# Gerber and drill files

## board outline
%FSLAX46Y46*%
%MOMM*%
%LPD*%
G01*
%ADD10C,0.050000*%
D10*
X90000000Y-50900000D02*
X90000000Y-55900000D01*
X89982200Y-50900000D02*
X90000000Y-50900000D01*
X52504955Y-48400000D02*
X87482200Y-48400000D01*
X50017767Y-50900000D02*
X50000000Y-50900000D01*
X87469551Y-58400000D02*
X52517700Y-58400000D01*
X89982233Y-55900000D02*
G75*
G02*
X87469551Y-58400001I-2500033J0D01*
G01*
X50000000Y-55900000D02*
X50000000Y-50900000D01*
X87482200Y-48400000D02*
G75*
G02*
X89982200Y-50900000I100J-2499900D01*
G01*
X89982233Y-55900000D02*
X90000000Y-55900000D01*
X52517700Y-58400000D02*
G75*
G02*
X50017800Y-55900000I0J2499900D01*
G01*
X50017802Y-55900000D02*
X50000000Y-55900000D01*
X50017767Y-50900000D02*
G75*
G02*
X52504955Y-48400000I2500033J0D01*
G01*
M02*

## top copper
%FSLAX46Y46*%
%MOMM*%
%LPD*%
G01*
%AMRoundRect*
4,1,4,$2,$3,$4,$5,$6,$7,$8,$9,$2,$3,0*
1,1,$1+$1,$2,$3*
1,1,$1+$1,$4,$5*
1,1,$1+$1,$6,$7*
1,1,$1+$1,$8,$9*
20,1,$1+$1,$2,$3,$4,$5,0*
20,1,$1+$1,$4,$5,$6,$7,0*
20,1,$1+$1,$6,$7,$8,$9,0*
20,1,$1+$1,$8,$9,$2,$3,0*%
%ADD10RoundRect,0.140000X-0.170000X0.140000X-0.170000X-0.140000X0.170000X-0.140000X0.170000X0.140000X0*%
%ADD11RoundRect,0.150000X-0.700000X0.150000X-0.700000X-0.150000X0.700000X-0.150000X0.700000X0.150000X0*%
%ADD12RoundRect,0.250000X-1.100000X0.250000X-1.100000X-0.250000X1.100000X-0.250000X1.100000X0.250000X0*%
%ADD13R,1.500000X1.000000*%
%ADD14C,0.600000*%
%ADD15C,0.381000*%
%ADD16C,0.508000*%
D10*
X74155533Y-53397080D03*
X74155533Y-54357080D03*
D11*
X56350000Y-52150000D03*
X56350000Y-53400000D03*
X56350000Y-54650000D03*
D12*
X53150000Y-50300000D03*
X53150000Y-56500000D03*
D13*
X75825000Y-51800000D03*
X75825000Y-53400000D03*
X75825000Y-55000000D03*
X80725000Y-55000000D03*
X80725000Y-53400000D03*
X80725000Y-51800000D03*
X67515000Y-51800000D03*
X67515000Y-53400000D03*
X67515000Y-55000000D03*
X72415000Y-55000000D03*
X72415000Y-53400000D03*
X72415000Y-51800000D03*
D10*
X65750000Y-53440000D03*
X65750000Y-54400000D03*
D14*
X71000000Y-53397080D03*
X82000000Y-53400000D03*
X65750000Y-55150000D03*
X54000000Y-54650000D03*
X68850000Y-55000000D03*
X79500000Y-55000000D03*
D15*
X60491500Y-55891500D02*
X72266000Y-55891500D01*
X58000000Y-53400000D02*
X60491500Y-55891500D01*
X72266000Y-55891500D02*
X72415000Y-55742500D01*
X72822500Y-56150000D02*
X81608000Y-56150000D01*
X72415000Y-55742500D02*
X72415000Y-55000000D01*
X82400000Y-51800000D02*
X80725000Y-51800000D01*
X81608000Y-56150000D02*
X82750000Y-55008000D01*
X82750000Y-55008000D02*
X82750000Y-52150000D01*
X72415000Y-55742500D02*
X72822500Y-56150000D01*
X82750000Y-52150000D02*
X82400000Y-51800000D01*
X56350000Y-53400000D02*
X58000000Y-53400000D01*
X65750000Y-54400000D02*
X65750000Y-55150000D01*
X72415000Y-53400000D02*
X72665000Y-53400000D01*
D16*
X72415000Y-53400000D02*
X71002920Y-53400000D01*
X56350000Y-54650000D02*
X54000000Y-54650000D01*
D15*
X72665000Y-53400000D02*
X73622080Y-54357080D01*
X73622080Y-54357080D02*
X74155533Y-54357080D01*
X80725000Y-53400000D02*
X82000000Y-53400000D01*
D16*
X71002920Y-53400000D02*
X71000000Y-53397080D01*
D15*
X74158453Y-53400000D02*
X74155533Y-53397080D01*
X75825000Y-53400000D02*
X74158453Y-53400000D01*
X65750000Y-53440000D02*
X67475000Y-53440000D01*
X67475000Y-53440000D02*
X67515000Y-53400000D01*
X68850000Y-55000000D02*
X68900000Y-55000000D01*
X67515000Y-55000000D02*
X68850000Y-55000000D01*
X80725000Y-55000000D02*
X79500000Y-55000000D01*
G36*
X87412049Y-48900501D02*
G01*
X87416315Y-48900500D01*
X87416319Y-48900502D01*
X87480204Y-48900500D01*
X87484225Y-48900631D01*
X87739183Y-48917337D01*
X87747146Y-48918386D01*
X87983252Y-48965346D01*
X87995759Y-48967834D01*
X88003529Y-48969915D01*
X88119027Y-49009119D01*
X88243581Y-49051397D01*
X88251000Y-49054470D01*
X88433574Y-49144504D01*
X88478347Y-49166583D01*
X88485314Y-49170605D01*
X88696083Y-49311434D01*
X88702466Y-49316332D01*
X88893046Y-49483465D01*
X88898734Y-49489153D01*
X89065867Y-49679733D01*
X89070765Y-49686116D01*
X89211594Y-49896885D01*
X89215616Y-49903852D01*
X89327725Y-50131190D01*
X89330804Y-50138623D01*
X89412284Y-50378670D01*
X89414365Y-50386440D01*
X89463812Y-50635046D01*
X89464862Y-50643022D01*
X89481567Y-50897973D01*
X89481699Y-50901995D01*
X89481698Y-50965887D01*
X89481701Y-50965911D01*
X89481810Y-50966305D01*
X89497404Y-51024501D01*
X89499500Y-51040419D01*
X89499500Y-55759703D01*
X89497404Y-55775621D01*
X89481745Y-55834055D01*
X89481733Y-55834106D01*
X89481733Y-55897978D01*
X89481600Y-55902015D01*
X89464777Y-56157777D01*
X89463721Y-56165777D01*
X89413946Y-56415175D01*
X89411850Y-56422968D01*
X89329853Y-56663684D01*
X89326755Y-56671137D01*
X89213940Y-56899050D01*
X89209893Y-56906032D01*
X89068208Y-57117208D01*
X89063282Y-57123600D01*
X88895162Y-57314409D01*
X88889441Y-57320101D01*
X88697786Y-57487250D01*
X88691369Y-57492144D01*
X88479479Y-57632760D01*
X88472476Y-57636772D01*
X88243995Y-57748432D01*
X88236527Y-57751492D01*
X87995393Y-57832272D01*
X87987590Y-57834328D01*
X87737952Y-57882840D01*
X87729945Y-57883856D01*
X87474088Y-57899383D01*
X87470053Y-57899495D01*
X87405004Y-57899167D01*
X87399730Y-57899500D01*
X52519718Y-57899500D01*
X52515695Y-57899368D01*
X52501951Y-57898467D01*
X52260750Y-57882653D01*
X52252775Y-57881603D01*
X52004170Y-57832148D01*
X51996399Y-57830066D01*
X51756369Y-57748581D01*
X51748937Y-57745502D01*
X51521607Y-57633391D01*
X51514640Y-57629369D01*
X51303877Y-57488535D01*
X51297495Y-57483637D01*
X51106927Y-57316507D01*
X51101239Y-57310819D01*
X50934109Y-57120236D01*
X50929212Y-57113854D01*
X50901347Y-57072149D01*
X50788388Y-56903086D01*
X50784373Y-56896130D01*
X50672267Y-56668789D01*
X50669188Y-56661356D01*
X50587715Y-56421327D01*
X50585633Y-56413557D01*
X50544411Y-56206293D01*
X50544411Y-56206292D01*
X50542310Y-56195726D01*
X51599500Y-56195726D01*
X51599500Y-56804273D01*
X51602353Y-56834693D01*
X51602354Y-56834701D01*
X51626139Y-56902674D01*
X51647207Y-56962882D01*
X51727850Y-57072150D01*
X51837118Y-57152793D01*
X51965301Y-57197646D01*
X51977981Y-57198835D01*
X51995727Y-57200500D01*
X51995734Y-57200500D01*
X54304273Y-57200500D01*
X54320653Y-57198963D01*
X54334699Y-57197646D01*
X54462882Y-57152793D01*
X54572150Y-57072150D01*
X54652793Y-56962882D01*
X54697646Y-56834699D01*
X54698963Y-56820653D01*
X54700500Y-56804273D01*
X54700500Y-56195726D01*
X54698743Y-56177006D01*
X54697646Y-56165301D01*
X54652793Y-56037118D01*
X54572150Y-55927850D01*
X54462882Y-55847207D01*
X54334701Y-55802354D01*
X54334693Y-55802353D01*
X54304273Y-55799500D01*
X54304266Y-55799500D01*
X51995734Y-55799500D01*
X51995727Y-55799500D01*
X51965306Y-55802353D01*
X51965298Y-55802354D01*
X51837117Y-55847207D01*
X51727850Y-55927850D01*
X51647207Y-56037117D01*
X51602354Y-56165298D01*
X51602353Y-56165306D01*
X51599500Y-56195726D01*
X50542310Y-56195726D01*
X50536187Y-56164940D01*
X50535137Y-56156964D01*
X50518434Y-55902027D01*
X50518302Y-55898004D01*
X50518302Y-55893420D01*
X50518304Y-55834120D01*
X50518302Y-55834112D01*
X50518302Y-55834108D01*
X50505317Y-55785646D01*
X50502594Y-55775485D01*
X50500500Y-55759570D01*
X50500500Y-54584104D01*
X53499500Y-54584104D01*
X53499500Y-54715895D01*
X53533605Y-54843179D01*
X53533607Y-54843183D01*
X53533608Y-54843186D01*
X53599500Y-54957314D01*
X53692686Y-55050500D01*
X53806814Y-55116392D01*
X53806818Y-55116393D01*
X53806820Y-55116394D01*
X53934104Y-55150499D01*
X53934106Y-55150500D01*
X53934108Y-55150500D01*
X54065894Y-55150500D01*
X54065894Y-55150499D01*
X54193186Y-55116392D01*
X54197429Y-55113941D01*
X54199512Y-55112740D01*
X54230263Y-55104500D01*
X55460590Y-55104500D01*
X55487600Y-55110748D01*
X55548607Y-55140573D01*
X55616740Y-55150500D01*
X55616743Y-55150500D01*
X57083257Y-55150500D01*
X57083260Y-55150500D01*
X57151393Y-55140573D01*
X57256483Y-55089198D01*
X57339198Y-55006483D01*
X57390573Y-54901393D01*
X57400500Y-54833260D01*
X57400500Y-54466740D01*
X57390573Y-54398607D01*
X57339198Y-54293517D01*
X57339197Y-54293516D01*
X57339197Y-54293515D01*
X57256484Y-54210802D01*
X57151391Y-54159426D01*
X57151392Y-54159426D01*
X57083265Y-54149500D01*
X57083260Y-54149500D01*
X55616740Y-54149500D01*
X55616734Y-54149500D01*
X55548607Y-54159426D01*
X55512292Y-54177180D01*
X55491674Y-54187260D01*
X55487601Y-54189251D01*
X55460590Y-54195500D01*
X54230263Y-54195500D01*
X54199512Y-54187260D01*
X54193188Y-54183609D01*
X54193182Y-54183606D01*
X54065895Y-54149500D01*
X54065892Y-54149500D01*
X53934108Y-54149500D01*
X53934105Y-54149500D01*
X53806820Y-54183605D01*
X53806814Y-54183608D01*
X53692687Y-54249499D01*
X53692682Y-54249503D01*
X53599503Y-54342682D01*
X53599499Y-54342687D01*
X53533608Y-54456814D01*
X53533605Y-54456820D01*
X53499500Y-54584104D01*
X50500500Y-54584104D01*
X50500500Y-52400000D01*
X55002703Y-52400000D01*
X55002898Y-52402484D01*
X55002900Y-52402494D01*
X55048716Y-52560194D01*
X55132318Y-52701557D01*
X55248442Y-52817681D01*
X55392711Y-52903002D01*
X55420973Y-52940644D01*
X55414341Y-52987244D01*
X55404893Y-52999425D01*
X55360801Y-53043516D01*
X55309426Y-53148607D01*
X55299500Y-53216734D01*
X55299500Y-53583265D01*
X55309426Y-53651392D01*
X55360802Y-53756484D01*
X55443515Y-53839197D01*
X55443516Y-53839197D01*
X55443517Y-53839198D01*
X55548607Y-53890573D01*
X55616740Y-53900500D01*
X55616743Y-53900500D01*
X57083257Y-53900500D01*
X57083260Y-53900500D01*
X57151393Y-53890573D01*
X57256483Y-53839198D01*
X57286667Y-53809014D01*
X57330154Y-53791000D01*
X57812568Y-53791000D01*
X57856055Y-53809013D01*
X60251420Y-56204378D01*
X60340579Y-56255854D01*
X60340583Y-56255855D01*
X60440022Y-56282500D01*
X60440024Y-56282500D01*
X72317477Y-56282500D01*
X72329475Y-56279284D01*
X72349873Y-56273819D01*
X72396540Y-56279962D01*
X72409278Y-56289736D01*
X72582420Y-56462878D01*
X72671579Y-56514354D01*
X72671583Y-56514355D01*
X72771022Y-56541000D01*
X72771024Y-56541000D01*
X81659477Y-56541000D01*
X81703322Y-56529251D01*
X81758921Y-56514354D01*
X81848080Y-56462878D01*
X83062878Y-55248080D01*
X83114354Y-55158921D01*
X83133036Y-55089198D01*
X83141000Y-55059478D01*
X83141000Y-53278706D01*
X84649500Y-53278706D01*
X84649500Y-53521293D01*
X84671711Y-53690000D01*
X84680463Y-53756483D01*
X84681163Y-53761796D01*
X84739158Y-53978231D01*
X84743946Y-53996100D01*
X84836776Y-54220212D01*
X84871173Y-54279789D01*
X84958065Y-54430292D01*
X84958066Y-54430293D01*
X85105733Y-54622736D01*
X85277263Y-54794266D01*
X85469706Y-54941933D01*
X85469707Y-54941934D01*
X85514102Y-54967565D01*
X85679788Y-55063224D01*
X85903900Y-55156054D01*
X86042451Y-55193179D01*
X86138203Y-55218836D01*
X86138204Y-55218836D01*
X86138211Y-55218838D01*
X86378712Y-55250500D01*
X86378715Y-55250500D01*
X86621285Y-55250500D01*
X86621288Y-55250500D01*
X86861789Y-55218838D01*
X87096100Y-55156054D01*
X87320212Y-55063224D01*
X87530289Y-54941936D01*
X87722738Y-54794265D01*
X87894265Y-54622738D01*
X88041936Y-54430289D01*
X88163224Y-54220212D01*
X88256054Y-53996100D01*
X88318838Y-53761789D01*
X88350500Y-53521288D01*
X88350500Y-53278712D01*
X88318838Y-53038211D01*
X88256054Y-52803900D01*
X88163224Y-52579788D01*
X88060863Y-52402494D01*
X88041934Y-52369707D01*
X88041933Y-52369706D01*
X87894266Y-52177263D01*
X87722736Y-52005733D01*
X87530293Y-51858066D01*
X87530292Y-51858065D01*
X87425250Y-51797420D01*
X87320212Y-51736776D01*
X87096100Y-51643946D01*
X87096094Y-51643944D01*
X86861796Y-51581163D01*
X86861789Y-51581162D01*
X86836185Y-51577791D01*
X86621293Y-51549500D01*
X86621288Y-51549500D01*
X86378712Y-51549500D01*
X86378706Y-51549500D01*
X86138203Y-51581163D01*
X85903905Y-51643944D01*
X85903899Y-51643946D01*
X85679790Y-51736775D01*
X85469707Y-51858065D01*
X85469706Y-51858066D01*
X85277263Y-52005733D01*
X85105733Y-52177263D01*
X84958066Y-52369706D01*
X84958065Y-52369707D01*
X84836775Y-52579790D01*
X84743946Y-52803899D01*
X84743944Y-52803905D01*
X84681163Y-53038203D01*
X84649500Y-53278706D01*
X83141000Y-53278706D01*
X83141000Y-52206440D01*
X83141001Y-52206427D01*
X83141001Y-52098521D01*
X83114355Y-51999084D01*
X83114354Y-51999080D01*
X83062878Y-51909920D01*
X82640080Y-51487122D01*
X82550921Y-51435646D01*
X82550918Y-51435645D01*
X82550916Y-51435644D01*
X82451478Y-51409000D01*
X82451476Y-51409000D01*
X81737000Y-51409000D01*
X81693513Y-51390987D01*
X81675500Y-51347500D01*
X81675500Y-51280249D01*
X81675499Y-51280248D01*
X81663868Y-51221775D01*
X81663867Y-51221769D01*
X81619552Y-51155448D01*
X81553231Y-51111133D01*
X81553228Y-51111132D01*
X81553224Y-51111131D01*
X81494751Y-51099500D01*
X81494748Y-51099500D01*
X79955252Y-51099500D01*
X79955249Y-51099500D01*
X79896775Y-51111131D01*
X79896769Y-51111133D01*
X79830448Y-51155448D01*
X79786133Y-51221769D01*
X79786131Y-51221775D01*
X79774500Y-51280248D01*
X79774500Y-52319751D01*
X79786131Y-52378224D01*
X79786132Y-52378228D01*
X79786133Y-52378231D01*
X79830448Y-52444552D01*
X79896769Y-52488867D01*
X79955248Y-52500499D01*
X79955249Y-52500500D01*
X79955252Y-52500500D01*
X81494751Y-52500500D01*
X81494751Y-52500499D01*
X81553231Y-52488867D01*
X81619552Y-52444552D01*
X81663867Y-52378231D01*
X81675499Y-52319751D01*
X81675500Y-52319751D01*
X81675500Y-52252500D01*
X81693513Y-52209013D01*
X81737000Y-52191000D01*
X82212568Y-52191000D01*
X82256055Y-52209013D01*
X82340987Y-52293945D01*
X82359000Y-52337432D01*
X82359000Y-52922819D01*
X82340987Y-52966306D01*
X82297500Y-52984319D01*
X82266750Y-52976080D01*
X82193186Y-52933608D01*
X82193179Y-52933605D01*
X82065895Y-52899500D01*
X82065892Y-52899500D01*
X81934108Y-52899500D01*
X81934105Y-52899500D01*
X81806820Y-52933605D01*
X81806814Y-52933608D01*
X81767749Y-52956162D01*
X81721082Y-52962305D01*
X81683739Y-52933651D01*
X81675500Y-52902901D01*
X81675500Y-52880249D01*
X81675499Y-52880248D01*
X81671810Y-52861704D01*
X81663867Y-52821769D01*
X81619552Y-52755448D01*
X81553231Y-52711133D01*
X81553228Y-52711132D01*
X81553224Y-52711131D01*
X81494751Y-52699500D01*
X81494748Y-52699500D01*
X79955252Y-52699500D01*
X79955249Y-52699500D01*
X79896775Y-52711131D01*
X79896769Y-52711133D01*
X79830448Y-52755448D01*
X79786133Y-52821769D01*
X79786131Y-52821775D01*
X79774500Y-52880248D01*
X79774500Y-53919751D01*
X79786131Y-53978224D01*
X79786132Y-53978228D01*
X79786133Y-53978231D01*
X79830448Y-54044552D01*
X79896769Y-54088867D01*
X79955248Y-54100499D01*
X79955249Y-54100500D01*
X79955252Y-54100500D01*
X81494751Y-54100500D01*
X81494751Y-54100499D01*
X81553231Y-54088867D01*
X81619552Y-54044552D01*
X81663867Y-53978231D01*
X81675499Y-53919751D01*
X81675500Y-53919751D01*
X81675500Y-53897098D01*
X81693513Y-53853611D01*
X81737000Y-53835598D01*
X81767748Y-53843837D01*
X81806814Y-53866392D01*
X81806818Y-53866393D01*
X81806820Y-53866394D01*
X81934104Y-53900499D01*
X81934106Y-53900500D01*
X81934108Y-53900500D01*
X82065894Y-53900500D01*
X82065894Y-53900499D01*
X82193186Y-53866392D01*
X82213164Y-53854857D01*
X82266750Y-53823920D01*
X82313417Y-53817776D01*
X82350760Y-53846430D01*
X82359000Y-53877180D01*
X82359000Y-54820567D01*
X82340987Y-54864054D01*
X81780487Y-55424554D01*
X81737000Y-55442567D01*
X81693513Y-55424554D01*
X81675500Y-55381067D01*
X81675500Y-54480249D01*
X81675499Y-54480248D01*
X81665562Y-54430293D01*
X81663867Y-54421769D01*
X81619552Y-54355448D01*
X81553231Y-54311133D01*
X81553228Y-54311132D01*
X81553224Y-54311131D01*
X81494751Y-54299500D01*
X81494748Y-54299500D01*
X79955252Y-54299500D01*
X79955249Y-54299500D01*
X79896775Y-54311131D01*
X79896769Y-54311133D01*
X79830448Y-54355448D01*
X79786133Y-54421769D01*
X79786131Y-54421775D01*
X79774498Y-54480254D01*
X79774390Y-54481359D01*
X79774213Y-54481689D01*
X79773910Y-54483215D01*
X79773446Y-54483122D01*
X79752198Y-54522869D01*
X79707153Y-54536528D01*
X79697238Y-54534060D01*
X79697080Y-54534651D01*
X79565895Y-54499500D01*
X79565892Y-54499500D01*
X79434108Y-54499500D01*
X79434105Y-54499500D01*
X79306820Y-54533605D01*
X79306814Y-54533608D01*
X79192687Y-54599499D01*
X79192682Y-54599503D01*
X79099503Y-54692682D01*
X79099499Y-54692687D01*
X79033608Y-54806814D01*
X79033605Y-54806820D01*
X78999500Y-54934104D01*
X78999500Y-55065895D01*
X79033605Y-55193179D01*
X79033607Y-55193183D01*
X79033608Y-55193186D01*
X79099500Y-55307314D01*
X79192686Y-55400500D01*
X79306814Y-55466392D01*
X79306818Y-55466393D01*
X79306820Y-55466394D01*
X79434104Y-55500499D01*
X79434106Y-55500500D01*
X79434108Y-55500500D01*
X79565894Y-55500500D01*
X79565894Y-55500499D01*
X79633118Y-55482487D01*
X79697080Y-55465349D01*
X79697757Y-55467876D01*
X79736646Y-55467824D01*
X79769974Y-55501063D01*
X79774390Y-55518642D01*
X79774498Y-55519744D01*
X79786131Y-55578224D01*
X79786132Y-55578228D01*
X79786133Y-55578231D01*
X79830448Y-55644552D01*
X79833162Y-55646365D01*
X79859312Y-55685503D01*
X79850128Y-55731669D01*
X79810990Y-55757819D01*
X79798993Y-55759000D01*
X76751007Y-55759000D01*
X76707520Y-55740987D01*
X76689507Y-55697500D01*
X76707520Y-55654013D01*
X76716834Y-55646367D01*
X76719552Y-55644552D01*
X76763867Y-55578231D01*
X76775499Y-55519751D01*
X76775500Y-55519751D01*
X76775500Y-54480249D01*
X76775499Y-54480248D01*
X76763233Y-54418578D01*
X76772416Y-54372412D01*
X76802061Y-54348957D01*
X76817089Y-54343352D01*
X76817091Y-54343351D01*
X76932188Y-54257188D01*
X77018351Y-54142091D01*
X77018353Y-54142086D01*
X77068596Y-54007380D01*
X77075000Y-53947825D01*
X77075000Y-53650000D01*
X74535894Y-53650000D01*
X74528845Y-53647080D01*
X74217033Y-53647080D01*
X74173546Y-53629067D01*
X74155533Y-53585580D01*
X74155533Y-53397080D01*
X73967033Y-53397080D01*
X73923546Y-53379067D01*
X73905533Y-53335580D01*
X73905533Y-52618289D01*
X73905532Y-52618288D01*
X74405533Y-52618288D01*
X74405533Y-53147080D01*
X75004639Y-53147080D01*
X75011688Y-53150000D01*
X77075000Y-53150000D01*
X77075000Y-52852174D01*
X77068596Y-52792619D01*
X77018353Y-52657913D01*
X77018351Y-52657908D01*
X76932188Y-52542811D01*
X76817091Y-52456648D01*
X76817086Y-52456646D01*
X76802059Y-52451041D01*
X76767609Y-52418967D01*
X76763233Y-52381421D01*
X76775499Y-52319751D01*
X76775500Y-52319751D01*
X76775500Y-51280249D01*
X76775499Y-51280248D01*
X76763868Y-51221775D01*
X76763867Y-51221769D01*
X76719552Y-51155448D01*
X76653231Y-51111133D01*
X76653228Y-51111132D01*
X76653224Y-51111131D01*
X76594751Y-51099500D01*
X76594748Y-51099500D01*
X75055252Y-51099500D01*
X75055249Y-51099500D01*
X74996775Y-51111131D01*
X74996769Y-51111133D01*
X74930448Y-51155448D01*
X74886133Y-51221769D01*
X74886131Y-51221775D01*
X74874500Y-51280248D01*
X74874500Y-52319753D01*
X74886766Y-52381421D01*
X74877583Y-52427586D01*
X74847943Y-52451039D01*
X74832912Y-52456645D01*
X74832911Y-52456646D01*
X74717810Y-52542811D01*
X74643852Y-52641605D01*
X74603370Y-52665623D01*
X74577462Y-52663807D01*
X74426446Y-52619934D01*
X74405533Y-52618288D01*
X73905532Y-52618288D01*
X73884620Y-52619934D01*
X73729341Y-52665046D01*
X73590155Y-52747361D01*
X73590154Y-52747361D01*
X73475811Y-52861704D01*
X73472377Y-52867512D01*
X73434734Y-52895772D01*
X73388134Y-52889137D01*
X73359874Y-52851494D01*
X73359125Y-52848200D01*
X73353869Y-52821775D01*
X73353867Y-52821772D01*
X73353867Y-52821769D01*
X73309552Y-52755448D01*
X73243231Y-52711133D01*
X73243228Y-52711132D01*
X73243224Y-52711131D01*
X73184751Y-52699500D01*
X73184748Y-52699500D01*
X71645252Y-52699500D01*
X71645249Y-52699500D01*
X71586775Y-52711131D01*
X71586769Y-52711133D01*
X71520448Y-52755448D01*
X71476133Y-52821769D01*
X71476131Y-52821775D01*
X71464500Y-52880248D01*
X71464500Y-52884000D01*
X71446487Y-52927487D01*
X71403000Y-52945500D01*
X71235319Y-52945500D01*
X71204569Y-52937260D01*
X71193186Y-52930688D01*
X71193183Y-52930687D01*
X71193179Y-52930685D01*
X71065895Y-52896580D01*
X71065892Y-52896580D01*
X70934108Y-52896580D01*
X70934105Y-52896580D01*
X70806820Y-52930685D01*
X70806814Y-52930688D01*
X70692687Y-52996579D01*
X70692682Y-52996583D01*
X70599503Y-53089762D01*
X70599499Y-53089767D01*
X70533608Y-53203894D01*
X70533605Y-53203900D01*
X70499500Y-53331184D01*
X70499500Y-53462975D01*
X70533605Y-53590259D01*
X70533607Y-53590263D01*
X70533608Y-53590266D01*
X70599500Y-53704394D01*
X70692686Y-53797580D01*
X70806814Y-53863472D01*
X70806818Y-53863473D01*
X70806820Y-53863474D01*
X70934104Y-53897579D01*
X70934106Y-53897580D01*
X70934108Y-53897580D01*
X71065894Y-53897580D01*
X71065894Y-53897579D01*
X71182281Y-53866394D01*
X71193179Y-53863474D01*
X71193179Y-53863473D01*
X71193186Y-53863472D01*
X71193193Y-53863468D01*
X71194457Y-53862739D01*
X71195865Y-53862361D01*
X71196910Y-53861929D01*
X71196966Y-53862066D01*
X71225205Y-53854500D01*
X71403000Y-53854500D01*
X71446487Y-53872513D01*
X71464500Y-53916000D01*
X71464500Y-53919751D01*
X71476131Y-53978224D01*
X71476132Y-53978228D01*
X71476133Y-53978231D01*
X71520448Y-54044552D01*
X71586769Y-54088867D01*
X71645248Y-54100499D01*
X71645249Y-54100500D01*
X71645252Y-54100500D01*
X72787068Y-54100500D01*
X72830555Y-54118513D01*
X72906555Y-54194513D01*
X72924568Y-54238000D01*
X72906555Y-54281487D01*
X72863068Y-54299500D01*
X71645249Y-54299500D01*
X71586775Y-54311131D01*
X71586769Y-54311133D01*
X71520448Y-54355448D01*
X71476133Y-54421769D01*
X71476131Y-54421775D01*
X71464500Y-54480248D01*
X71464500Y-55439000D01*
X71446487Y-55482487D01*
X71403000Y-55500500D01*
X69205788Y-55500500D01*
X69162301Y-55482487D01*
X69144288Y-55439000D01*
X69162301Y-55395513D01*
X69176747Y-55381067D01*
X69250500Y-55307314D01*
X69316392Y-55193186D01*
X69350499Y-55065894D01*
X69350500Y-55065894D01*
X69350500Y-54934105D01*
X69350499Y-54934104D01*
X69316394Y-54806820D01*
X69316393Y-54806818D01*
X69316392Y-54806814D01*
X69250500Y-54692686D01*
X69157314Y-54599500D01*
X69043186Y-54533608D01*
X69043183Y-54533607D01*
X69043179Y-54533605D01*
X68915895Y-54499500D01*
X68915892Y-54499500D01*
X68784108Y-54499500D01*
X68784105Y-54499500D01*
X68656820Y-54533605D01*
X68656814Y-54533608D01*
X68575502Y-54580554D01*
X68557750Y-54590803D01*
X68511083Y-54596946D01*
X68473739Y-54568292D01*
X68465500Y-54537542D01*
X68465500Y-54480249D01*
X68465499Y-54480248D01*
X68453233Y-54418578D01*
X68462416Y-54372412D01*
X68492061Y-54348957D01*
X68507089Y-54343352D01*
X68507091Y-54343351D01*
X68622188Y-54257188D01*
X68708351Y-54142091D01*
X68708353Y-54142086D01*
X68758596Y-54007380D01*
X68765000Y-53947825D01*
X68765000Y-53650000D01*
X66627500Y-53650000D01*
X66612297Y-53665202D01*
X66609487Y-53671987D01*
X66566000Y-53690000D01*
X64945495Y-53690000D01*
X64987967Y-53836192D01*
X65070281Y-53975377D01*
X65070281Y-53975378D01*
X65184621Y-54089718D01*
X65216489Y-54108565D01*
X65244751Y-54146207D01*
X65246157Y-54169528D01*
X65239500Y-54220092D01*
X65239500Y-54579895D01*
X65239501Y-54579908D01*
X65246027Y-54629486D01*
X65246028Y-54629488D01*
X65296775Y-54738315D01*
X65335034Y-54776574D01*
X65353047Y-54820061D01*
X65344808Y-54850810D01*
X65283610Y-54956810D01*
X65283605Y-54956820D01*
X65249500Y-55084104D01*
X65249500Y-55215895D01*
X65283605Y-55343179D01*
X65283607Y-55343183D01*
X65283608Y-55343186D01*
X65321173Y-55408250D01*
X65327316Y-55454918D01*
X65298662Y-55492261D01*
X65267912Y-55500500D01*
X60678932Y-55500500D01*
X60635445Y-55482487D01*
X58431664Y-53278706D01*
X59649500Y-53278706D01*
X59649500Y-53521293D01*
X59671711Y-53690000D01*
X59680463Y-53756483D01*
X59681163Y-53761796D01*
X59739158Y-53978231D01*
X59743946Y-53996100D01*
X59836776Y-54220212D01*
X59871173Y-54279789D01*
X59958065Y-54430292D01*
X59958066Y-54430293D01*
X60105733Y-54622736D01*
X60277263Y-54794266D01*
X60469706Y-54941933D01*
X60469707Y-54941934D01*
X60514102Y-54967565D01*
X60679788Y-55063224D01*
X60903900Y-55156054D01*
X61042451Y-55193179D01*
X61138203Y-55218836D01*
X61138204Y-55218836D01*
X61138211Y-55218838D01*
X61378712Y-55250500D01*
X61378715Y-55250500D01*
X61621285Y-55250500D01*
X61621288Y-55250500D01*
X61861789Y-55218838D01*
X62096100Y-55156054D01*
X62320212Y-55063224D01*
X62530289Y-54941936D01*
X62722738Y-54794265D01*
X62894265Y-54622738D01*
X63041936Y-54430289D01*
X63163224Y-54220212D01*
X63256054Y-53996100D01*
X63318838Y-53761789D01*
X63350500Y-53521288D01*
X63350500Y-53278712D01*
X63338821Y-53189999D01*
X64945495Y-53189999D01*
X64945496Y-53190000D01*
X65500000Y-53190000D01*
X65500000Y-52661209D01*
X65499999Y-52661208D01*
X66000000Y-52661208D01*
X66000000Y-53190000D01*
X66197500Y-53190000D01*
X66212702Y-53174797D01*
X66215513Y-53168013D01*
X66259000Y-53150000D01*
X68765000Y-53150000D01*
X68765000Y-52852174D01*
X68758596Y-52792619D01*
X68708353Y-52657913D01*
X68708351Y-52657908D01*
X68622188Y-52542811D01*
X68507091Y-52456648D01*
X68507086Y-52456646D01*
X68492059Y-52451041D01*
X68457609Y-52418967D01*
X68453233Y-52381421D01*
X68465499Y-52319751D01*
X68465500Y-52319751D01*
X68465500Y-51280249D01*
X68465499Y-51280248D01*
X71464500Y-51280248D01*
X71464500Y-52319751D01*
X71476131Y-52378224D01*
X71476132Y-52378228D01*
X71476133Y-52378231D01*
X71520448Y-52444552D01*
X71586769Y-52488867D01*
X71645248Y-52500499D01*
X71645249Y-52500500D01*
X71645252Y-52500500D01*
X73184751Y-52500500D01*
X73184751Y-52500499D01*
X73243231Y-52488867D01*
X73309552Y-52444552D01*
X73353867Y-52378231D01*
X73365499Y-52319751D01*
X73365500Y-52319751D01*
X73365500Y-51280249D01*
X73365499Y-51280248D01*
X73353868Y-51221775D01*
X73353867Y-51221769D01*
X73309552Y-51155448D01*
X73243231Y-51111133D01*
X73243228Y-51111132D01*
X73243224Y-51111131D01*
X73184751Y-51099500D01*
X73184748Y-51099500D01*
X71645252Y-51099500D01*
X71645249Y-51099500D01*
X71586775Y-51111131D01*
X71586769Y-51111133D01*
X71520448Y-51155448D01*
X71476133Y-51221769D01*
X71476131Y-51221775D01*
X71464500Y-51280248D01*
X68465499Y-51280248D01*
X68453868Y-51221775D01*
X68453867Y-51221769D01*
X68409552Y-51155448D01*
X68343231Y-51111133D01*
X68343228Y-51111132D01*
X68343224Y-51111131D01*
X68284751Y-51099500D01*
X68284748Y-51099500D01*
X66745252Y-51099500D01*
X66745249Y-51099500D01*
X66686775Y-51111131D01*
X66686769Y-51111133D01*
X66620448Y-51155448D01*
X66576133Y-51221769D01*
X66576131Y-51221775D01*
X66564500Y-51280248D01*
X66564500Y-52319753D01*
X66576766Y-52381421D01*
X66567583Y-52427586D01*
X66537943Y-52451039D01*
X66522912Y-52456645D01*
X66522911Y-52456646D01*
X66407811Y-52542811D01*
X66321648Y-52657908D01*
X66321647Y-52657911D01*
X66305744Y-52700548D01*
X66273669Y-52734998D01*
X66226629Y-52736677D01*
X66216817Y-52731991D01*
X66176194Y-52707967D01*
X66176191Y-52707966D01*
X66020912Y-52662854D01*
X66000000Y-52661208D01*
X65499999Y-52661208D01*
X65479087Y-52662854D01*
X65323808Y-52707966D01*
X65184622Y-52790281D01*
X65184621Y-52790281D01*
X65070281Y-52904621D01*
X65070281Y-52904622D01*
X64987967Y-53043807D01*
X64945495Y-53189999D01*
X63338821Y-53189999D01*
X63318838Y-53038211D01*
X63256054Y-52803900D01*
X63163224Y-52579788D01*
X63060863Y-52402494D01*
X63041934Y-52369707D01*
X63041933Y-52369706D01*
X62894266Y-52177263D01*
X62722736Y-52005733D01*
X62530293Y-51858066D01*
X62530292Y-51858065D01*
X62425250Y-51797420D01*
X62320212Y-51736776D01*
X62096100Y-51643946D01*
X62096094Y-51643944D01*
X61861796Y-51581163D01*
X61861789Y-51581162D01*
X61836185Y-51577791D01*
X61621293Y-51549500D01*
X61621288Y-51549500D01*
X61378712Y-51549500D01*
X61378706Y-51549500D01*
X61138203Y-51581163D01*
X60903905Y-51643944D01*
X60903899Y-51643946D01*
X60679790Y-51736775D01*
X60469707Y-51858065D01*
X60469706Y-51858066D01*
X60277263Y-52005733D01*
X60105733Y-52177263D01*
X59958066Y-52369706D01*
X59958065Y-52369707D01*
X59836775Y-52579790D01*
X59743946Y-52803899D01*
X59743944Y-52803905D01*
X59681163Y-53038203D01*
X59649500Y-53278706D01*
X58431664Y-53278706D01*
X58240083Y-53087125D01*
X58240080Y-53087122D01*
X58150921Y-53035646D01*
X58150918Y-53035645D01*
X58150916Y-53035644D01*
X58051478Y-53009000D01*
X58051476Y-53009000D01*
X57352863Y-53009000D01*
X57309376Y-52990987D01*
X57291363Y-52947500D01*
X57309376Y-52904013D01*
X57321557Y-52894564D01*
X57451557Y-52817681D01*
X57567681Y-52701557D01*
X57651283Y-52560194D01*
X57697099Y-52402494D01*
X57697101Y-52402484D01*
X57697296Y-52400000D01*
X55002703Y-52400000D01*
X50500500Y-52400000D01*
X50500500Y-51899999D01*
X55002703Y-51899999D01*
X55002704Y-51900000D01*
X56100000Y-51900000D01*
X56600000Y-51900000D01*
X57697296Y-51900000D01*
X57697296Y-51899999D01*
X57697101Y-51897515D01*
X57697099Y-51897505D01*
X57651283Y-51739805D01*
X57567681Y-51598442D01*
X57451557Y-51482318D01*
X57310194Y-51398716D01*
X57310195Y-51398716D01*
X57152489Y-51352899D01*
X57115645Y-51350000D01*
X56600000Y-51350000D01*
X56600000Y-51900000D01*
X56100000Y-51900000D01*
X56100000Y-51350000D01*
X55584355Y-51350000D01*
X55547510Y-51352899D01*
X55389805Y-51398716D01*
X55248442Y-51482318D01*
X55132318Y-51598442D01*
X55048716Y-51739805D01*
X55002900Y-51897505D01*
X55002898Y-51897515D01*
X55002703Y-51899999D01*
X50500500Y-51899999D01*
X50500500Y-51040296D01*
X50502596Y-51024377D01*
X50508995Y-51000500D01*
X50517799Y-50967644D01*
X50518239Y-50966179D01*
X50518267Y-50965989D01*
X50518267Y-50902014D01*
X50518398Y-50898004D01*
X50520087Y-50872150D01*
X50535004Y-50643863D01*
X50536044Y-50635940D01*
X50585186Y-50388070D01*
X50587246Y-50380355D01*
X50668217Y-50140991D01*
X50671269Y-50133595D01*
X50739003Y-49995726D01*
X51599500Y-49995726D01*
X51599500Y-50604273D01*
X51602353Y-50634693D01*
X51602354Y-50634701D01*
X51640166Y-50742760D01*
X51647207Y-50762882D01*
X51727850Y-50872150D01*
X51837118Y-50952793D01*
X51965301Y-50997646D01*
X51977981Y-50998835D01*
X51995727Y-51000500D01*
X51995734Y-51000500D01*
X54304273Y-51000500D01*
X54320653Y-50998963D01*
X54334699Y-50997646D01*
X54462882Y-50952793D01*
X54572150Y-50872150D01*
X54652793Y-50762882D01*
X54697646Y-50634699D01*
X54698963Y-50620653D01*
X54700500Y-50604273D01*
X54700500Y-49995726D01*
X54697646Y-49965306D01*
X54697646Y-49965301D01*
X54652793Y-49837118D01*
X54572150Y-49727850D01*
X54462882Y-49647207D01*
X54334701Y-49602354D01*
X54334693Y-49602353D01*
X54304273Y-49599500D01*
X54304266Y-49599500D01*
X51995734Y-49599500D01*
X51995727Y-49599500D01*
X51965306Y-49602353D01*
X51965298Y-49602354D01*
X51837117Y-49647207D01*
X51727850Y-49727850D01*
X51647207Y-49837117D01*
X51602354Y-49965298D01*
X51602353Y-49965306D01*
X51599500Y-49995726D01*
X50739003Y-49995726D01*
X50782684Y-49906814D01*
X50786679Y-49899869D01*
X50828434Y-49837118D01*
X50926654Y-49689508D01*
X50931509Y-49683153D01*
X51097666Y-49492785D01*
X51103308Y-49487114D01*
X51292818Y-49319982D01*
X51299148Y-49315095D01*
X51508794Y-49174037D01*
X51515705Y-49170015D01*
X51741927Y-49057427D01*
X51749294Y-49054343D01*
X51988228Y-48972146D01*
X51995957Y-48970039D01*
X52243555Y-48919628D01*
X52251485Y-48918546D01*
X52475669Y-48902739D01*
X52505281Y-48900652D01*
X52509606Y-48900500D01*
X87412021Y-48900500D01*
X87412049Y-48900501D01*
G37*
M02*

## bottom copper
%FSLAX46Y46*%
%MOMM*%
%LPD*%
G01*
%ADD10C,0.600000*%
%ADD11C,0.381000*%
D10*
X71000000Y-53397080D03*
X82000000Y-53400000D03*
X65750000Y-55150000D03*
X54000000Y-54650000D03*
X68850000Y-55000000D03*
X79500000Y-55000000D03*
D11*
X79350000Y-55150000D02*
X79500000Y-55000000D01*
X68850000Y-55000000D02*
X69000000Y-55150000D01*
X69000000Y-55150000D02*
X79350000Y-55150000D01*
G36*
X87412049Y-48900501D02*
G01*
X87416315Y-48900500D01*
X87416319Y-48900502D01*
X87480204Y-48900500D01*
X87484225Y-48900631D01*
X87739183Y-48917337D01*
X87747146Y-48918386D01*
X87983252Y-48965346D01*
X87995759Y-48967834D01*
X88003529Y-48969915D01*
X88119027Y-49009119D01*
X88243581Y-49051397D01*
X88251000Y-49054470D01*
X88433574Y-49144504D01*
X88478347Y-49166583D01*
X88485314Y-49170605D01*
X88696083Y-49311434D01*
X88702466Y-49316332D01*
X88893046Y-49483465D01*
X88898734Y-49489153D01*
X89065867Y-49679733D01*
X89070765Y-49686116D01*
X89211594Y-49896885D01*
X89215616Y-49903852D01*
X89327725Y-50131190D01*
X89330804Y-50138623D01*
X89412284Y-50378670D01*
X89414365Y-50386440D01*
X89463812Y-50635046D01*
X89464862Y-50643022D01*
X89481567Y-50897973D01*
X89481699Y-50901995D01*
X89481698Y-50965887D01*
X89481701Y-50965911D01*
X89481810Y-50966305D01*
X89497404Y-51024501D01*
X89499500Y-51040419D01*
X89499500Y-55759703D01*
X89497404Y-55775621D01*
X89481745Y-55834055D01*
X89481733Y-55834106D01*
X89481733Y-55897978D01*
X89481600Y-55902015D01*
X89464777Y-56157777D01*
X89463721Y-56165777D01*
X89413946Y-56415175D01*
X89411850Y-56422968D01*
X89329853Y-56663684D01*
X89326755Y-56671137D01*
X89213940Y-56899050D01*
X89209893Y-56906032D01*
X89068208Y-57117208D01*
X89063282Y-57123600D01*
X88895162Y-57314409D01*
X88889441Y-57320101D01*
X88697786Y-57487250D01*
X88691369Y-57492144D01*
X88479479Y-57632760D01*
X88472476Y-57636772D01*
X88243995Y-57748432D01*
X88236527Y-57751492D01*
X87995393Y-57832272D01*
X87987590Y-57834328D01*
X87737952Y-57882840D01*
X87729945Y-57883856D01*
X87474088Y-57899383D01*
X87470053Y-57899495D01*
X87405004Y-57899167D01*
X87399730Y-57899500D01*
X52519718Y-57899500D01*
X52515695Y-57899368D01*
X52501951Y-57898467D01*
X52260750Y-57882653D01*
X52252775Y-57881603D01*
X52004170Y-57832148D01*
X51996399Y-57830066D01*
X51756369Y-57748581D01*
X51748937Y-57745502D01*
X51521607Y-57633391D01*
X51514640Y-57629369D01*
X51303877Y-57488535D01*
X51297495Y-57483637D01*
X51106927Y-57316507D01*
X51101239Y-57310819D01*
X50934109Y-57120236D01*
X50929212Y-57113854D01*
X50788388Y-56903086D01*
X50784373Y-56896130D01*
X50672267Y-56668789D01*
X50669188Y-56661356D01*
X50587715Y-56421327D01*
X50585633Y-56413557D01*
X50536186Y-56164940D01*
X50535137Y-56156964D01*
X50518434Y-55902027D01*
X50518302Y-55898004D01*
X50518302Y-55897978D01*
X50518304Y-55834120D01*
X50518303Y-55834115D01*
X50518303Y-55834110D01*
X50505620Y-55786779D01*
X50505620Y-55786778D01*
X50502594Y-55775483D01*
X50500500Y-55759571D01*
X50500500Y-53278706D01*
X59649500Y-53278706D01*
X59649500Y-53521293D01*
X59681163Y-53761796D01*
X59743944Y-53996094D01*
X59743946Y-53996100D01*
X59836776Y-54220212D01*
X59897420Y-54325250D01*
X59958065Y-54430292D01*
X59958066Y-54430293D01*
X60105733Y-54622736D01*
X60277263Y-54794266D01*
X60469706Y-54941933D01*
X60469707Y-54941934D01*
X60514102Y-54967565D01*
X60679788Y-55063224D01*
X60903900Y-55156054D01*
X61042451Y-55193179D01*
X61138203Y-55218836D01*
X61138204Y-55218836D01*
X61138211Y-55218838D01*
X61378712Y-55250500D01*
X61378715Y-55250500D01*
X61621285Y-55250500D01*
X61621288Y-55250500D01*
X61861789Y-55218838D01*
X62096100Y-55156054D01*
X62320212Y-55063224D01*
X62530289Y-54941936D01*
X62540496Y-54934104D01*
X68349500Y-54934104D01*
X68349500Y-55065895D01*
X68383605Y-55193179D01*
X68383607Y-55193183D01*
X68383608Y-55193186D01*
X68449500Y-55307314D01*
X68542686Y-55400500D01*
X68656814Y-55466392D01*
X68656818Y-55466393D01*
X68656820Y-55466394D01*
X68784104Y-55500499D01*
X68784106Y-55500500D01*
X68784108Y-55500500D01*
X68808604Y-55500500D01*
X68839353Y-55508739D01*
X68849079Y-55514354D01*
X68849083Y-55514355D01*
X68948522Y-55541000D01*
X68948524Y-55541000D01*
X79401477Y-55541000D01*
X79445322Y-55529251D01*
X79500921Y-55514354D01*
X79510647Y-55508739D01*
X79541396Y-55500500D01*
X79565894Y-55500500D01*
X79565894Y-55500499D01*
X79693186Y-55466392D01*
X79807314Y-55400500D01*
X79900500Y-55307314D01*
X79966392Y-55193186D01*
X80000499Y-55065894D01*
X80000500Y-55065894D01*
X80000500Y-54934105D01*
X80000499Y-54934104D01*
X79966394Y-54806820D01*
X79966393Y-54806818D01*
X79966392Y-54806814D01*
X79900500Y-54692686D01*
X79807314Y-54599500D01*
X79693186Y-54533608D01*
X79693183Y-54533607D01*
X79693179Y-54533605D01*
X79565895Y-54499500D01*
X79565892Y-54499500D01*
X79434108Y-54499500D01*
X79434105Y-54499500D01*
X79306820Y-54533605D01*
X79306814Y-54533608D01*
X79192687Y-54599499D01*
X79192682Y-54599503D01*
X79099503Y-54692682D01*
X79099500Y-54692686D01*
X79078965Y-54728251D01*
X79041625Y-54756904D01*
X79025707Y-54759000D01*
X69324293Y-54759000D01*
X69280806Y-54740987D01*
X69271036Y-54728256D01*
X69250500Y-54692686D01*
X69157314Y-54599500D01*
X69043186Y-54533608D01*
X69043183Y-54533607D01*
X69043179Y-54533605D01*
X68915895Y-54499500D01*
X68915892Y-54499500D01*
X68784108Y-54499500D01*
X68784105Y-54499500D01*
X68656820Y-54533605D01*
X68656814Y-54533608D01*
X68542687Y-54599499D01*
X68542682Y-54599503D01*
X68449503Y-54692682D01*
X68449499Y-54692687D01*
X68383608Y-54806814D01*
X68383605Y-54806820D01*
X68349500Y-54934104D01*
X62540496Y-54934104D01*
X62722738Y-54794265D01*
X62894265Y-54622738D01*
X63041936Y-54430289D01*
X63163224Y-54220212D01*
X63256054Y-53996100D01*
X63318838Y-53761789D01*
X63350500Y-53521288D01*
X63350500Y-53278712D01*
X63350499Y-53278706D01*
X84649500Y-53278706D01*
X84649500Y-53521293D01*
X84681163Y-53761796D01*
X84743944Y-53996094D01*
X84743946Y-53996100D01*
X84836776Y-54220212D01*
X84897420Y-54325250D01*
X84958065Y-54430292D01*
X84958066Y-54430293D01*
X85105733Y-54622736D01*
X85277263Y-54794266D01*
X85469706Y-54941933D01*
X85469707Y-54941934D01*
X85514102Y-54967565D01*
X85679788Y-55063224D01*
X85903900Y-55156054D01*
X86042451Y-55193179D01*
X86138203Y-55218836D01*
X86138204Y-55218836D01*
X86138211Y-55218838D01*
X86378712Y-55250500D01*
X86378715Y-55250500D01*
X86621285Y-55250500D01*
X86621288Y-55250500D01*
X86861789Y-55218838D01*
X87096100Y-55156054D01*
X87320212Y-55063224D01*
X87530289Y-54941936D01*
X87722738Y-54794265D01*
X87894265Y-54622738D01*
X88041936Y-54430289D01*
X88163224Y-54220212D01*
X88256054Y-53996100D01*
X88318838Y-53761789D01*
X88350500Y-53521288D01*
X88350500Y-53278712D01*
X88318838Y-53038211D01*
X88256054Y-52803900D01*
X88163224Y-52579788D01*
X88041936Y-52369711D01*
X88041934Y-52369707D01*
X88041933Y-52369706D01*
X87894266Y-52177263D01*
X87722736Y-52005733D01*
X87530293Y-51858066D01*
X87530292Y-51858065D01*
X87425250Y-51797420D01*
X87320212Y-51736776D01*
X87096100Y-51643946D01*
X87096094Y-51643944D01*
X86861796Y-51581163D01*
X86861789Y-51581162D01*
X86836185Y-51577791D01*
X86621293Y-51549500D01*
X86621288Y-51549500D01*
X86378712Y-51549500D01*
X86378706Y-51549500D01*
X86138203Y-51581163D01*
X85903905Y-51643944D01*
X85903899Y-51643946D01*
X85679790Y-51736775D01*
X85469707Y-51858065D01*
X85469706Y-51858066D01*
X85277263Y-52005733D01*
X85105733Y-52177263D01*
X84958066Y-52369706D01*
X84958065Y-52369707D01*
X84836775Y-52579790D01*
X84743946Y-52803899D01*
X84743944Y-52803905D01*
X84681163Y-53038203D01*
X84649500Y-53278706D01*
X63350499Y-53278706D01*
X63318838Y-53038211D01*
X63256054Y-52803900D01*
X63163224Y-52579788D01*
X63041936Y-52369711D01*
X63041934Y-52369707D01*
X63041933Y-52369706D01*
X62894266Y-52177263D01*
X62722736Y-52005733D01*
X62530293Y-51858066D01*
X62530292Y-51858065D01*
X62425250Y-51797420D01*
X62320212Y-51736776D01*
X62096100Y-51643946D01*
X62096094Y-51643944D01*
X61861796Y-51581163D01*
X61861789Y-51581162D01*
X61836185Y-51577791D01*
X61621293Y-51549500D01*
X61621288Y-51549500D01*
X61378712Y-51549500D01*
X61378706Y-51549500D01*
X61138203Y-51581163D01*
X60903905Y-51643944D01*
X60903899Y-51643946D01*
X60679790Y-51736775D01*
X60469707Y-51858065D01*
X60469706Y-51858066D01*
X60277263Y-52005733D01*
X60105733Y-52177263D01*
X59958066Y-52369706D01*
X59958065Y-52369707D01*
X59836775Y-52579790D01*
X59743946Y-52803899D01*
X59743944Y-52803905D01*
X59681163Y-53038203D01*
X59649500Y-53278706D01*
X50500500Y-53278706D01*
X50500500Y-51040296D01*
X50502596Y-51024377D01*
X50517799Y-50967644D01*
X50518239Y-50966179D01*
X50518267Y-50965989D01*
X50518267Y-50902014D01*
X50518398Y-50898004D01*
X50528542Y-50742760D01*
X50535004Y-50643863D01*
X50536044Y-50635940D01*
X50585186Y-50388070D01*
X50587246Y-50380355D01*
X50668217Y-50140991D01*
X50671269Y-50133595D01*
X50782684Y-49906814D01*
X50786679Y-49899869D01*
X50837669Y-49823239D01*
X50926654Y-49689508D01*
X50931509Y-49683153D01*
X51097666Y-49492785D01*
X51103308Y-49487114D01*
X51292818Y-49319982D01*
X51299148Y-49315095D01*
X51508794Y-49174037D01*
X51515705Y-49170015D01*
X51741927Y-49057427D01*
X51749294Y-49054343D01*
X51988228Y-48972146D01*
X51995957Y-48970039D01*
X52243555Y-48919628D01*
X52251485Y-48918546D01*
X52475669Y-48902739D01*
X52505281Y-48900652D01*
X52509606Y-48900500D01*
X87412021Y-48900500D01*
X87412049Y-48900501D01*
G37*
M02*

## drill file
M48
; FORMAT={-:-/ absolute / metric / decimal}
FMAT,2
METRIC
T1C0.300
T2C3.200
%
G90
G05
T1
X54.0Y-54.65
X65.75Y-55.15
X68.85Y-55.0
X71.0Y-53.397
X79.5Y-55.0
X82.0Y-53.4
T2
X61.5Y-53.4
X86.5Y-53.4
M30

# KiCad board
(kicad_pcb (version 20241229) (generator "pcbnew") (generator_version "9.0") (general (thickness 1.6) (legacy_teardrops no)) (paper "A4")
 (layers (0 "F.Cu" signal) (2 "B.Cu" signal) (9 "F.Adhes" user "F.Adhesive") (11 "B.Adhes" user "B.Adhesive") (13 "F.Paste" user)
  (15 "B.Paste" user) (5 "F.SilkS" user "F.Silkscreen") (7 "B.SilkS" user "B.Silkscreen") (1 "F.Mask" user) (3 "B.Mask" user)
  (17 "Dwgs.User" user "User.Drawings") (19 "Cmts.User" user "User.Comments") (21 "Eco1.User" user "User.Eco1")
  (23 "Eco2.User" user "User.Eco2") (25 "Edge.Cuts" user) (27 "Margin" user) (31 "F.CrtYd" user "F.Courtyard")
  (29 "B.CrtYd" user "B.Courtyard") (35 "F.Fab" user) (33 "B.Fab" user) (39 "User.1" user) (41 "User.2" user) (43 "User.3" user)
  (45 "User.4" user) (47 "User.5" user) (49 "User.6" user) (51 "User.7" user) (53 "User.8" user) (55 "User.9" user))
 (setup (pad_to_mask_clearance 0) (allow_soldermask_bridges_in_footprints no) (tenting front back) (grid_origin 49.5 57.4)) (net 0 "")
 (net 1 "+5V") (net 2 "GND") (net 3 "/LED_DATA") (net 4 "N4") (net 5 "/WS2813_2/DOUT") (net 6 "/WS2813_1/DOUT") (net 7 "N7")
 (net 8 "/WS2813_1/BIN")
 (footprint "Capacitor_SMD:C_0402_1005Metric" (layer "F.Cu") (at 74.155533 53.87708 -90)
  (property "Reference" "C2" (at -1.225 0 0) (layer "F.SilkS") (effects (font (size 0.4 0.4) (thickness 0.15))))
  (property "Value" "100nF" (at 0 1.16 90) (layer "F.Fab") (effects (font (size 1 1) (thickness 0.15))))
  (pad "1" smd roundrect (at -0.48 0 270) (size 0.56 0.62) (layers "F.Cu" "F.Mask" "F.Paste") (roundrect_rratio 0.25) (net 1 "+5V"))
  (pad "2" smd roundrect (at 0.48 0 270) (size 0.56 0.62) (layers "F.Cu" "F.Mask" "F.Paste") (roundrect_rratio 0.25) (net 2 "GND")))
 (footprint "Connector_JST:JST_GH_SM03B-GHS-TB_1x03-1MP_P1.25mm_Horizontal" (layer "F.Cu") (at 54.5 53.4 -90)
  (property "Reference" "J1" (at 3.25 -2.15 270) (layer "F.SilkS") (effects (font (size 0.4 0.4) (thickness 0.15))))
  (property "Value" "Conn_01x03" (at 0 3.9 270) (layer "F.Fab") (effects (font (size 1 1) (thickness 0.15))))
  (pad "1" smd roundrect (at -1.25 -1.85 270) (size 0.6 1.7) (layers "F.Cu" "F.Mask" "F.Paste") (roundrect_rratio 0.25) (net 1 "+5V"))
  (pad "2" smd roundrect (at 0 -1.85 270) (size 0.6 1.7) (layers "F.Cu" "F.Mask" "F.Paste") (roundrect_rratio 0.25) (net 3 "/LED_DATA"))
  (pad "3" smd roundrect (at 1.25 -1.85 270) (size 0.6 1.7) (layers "F.Cu" "F.Mask" "F.Paste") (roundrect_rratio 0.25) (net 2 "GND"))
  (pad "MP" smd roundrect (at -3.1 1.35 270) (size 1 2.7) (layers "F.Cu" "F.Mask" "F.Paste") (roundrect_rratio 0.25))
  (pad "MP" smd roundrect (at 3.1 1.35 270) (size 1 2.7) (layers "F.Cu" "F.Mask" "F.Paste") (roundrect_rratio 0.25)))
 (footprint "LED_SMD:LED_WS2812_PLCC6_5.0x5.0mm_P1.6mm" (layer "F.Cu") (at 78.275 53.4)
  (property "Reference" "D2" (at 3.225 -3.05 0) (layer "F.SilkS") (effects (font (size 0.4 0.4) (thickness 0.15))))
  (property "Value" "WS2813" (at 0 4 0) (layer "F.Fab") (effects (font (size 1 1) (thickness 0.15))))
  (pad "1" smd rect (at -2.45 -1.6) (size 1.5 1) (layers "F.Cu" "F.Mask" "F.Paste") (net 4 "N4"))
  (pad "2" smd rect (at -2.45 0) (size 1.5 1) (layers "F.Cu" "F.Mask" "F.Paste") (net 1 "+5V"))
  (pad "3" smd rect (at -2.45 1.6) (size 1.5 1) (layers "F.Cu" "F.Mask" "F.Paste") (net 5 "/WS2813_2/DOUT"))
  (pad "4" smd rect (at 2.45 1.6) (size 1.5 1) (layers "F.Cu" "F.Mask" "F.Paste") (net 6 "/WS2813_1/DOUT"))
  (pad "5" smd rect (at 2.45 0) (size 1.5 1) (layers "F.Cu" "F.Mask" "F.Paste") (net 2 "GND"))
  (pad "6" smd rect (at 2.45 -1.6) (size 1.5 1) (layers "F.Cu" "F.Mask" "F.Paste") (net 3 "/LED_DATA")))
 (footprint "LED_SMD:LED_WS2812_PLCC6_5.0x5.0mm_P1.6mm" (layer "F.Cu") (at 69.965 53.4)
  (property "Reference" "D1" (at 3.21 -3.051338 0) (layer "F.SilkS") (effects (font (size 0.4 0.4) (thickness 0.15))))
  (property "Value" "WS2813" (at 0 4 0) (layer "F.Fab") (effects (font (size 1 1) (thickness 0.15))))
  (pad "1" smd rect (at -2.45 -1.6) (size 1.5 1) (layers "F.Cu" "F.Mask" "F.Paste") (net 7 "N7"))
  (pad "2" smd rect (at -2.45 0) (size 1.5 1) (layers "F.Cu" "F.Mask" "F.Paste") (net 1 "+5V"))
  (pad "3" smd rect (at -2.45 1.6) (size 1.5 1) (layers "F.Cu" "F.Mask" "F.Paste") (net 6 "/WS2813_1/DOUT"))
  (pad "4" smd rect (at 2.45 1.6) (size 1.5 1) (layers "F.Cu" "F.Mask" "F.Paste") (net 3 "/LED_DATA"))
  (pad "5" smd rect (at 2.45 0) (size 1.5 1) (layers "F.Cu" "F.Mask" "F.Paste") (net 2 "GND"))
  (pad "6" smd rect (at 2.45 -1.6) (size 1.5 1) (layers "F.Cu" "F.Mask" "F.Paste") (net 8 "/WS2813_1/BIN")))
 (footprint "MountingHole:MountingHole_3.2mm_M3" (layer "F.Cu") (at 61.5 53.4)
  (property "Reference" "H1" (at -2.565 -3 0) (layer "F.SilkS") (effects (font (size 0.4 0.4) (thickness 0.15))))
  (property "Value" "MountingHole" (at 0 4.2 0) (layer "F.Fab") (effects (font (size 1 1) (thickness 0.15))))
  (pad "" np_thru_hole circle (at 0 0) (size 3.2 3.2) (drill 3.2) (layers "*.Cu" "*.Mask")))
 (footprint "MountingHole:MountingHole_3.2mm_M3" (layer "F.Cu") (at 86.5 53.4)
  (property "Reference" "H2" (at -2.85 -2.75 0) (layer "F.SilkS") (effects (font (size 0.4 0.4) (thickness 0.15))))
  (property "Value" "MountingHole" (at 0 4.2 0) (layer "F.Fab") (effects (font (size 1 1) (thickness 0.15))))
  (pad "" np_thru_hole circle (at 0 0) (size 3.2 3.2) (drill 3.2) (layers "*.Cu" "*.Mask")))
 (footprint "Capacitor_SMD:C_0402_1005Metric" (layer "F.Cu") (at 65.75 53.92 -90)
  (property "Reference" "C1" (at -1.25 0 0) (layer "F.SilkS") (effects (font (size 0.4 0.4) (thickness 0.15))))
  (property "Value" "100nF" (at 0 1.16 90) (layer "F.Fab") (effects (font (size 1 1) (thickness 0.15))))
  (pad "1" smd roundrect (at -0.48 0 270) (size 0.56 0.62) (layers "F.Cu" "F.Mask" "F.Paste") (roundrect_rratio 0.25) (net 1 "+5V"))
  (pad "2" smd roundrect (at 0.48 0 270) (size 0.56 0.62) (layers "F.Cu" "F.Mask" "F.Paste") (roundrect_rratio 0.25) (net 2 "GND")))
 (gr_line (start 90 50.9) (end 90 55.9) (stroke (width 0.05) (type default)) (layer "Edge.Cuts"))
 (gr_line (start 89.9822 50.9) (end 90 50.9) (stroke (width 0.05) (type default)) (layer "Edge.Cuts"))
 (gr_line (start 52.504955 48.4) (end 87.4822 48.4) (stroke (width 0.05) (type default)) (layer "Edge.Cuts"))
 (gr_line (start 50.017767 50.9) (end 50 50.9) (stroke (width 0.05) (type default)) (layer "Edge.Cuts"))
 (gr_line (start 87.469551 58.4) (end 52.5177 58.4) (stroke (width 0.05) (type default)) (layer "Edge.Cuts"))
 (gr_arc (start 89.982233 55.9) (mid 89.25 57.667767) (end 87.469551 58.4) (stroke (width 0.05) (type default)) (layer "Edge.Cuts"))
 (gr_line (start 50 55.9) (end 50 50.9) (stroke (width 0.05) (type default)) (layer "Edge.Cuts"))
 (gr_arc (start 87.4822 48.4) (mid 89.25 49.132233) (end 89.9822 50.9) (stroke (width 0.05) (type default)) (layer "Edge.Cuts"))
 (gr_line (start 89.982233 55.9) (end 90 55.9) (stroke (width 0.05) (type default)) (layer "Edge.Cuts"))
 (gr_arc (start 52.5177 58.4) (mid 50.75 57.667767) (end 50.017802 55.9) (stroke (width 0.05) (type default)) (layer "Edge.Cuts"))
 (gr_line (start 50.017802 55.9) (end 50 55.9) (stroke (width 0.05) (type default)) (layer "Edge.Cuts"))
 (gr_arc (start 50.017767 50.9) (mid 50.75 49.132233) (end 52.504955 48.4) (stroke (width 0.05) (type default)) (layer "Edge.Cuts"))
 (segment (start 60.4915 55.8915) (end 72.266 55.8915) (width 0.381) (layer "F.Cu") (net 3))
 (segment (start 58 53.4) (end 60.4915 55.8915) (width 0.381) (layer "F.Cu") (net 3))
 (segment (start 72.266 55.8915) (end 72.415 55.7425) (width 0.381) (layer "F.Cu") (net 3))
 (segment (start 72.8225 56.15) (end 81.608 56.15) (width 0.381) (layer "F.Cu") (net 3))
 (segment (start 72.415 55.7425) (end 72.415 55) (width 0.381) (layer "F.Cu") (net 3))
 (segment (start 82.4 51.8) (end 80.725 51.8) (width 0.381) (layer "F.Cu") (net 3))
 (segment (start 81.608 56.15) (end 82.75 55.008) (width 0.381) (layer "F.Cu") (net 3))
 (segment (start 82.75 55.008) (end 82.75 52.15) (width 0.381) (layer "F.Cu") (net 3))
 (segment (start 72.415 55.7425) (end 72.8225 56.15) (width 0.381) (layer "F.Cu") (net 3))
 (segment (start 82.75 52.15) (end 82.4 51.8) (width 0.381) (layer "F.Cu") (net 3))
 (segment (start 56.35 53.4) (end 58 53.4) (width 0.381) (layer "F.Cu") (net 3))
 (segment (start 65.75 54.4) (end 65.75 55.15) (width 0.381) (layer "F.Cu") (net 2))
 (segment (start 72.415 53.4) (end 72.665 53.4) (width 0.381) (layer "F.Cu") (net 2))
 (segment (start 72.415 53.4) (end 71.00292 53.4) (width 0.508) (layer "F.Cu") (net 2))
 (segment (start 56.35 54.65) (end 54 54.65) (width 0.508) (layer "F.Cu") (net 2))
 (segment (start 72.665 53.4) (end 73.62208 54.35708) (width 0.381) (layer "F.Cu") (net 2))
 (segment (start 73.62208 54.35708) (end 74.155533 54.35708) (width 0.381) (layer "F.Cu") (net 2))
 (segment (start 80.725 53.4) (end 82 53.4) (width 0.381) (layer "F.Cu") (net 2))
 (segment (start 71.00292 53.4) (end 71 53.39708) (width 0.508) (layer "F.Cu") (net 2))
 (via (at 71 53.39708) (size 0.6) (drill 0.3) (layers "F.Cu" "B.Cu") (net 2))
 (via (at 82 53.4) (size 0.6) (drill 0.3) (layers "F.Cu" "B.Cu") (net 2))
 (via (at 65.75 55.15) (size 0.6) (drill 0.3) (layers "F.Cu" "B.Cu") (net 2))
 (via (at 54 54.65) (size 0.6) (drill 0.3) (layers "F.Cu" "B.Cu") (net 2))
 (segment (start 74.158453 53.4) (end 74.155533 53.39708) (width 0.381) (layer "F.Cu") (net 1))
 (segment (start 75.825 53.4) (end 74.158453 53.4) (width 0.381) (layer "F.Cu") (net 1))
 (segment (start 65.75 53.44) (end 67.475 53.44) (width 0.381) (layer "F.Cu") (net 1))
 (segment (start 67.475 53.44) (end 67.515 53.4) (width 0.381) (layer "F.Cu") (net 1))
 (segment (start 68.85 55) (end 68.9 55) (width 0.381) (layer "F.Cu") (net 6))
 (segment (start 67.515 55) (end 68.85 55) (width 0.381) (layer "F.Cu") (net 6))
 (segment (start 80.725 55) (end 79.5 55) (width 0.381) (layer "F.Cu") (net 6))
 (via (at 68.85 55) (size 0.6) (drill 0.3) (layers "F.Cu" "B.Cu") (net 6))
 (via (at 79.5 55) (size 0.6) (drill 0.3) (layers "F.Cu" "B.Cu") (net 6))
 (segment (start 79.35 55.15) (end 79.5 55) (width 0.381) (layer "B.Cu") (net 6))
 (segment (start 68.85 55) (end 69 55.15) (width 0.381) (layer "B.Cu") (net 6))
 (segment (start 69 55.15) (end 79.35 55.15) (width 0.381) (layer "B.Cu") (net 6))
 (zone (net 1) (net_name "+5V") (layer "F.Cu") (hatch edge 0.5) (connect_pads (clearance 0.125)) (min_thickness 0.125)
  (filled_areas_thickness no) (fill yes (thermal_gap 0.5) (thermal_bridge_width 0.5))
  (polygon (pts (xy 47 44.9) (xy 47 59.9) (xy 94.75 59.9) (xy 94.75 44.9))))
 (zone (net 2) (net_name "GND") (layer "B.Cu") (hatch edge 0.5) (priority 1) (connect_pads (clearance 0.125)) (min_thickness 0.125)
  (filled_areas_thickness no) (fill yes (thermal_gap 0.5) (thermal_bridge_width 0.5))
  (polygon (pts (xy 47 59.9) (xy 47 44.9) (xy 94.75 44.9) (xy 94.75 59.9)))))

